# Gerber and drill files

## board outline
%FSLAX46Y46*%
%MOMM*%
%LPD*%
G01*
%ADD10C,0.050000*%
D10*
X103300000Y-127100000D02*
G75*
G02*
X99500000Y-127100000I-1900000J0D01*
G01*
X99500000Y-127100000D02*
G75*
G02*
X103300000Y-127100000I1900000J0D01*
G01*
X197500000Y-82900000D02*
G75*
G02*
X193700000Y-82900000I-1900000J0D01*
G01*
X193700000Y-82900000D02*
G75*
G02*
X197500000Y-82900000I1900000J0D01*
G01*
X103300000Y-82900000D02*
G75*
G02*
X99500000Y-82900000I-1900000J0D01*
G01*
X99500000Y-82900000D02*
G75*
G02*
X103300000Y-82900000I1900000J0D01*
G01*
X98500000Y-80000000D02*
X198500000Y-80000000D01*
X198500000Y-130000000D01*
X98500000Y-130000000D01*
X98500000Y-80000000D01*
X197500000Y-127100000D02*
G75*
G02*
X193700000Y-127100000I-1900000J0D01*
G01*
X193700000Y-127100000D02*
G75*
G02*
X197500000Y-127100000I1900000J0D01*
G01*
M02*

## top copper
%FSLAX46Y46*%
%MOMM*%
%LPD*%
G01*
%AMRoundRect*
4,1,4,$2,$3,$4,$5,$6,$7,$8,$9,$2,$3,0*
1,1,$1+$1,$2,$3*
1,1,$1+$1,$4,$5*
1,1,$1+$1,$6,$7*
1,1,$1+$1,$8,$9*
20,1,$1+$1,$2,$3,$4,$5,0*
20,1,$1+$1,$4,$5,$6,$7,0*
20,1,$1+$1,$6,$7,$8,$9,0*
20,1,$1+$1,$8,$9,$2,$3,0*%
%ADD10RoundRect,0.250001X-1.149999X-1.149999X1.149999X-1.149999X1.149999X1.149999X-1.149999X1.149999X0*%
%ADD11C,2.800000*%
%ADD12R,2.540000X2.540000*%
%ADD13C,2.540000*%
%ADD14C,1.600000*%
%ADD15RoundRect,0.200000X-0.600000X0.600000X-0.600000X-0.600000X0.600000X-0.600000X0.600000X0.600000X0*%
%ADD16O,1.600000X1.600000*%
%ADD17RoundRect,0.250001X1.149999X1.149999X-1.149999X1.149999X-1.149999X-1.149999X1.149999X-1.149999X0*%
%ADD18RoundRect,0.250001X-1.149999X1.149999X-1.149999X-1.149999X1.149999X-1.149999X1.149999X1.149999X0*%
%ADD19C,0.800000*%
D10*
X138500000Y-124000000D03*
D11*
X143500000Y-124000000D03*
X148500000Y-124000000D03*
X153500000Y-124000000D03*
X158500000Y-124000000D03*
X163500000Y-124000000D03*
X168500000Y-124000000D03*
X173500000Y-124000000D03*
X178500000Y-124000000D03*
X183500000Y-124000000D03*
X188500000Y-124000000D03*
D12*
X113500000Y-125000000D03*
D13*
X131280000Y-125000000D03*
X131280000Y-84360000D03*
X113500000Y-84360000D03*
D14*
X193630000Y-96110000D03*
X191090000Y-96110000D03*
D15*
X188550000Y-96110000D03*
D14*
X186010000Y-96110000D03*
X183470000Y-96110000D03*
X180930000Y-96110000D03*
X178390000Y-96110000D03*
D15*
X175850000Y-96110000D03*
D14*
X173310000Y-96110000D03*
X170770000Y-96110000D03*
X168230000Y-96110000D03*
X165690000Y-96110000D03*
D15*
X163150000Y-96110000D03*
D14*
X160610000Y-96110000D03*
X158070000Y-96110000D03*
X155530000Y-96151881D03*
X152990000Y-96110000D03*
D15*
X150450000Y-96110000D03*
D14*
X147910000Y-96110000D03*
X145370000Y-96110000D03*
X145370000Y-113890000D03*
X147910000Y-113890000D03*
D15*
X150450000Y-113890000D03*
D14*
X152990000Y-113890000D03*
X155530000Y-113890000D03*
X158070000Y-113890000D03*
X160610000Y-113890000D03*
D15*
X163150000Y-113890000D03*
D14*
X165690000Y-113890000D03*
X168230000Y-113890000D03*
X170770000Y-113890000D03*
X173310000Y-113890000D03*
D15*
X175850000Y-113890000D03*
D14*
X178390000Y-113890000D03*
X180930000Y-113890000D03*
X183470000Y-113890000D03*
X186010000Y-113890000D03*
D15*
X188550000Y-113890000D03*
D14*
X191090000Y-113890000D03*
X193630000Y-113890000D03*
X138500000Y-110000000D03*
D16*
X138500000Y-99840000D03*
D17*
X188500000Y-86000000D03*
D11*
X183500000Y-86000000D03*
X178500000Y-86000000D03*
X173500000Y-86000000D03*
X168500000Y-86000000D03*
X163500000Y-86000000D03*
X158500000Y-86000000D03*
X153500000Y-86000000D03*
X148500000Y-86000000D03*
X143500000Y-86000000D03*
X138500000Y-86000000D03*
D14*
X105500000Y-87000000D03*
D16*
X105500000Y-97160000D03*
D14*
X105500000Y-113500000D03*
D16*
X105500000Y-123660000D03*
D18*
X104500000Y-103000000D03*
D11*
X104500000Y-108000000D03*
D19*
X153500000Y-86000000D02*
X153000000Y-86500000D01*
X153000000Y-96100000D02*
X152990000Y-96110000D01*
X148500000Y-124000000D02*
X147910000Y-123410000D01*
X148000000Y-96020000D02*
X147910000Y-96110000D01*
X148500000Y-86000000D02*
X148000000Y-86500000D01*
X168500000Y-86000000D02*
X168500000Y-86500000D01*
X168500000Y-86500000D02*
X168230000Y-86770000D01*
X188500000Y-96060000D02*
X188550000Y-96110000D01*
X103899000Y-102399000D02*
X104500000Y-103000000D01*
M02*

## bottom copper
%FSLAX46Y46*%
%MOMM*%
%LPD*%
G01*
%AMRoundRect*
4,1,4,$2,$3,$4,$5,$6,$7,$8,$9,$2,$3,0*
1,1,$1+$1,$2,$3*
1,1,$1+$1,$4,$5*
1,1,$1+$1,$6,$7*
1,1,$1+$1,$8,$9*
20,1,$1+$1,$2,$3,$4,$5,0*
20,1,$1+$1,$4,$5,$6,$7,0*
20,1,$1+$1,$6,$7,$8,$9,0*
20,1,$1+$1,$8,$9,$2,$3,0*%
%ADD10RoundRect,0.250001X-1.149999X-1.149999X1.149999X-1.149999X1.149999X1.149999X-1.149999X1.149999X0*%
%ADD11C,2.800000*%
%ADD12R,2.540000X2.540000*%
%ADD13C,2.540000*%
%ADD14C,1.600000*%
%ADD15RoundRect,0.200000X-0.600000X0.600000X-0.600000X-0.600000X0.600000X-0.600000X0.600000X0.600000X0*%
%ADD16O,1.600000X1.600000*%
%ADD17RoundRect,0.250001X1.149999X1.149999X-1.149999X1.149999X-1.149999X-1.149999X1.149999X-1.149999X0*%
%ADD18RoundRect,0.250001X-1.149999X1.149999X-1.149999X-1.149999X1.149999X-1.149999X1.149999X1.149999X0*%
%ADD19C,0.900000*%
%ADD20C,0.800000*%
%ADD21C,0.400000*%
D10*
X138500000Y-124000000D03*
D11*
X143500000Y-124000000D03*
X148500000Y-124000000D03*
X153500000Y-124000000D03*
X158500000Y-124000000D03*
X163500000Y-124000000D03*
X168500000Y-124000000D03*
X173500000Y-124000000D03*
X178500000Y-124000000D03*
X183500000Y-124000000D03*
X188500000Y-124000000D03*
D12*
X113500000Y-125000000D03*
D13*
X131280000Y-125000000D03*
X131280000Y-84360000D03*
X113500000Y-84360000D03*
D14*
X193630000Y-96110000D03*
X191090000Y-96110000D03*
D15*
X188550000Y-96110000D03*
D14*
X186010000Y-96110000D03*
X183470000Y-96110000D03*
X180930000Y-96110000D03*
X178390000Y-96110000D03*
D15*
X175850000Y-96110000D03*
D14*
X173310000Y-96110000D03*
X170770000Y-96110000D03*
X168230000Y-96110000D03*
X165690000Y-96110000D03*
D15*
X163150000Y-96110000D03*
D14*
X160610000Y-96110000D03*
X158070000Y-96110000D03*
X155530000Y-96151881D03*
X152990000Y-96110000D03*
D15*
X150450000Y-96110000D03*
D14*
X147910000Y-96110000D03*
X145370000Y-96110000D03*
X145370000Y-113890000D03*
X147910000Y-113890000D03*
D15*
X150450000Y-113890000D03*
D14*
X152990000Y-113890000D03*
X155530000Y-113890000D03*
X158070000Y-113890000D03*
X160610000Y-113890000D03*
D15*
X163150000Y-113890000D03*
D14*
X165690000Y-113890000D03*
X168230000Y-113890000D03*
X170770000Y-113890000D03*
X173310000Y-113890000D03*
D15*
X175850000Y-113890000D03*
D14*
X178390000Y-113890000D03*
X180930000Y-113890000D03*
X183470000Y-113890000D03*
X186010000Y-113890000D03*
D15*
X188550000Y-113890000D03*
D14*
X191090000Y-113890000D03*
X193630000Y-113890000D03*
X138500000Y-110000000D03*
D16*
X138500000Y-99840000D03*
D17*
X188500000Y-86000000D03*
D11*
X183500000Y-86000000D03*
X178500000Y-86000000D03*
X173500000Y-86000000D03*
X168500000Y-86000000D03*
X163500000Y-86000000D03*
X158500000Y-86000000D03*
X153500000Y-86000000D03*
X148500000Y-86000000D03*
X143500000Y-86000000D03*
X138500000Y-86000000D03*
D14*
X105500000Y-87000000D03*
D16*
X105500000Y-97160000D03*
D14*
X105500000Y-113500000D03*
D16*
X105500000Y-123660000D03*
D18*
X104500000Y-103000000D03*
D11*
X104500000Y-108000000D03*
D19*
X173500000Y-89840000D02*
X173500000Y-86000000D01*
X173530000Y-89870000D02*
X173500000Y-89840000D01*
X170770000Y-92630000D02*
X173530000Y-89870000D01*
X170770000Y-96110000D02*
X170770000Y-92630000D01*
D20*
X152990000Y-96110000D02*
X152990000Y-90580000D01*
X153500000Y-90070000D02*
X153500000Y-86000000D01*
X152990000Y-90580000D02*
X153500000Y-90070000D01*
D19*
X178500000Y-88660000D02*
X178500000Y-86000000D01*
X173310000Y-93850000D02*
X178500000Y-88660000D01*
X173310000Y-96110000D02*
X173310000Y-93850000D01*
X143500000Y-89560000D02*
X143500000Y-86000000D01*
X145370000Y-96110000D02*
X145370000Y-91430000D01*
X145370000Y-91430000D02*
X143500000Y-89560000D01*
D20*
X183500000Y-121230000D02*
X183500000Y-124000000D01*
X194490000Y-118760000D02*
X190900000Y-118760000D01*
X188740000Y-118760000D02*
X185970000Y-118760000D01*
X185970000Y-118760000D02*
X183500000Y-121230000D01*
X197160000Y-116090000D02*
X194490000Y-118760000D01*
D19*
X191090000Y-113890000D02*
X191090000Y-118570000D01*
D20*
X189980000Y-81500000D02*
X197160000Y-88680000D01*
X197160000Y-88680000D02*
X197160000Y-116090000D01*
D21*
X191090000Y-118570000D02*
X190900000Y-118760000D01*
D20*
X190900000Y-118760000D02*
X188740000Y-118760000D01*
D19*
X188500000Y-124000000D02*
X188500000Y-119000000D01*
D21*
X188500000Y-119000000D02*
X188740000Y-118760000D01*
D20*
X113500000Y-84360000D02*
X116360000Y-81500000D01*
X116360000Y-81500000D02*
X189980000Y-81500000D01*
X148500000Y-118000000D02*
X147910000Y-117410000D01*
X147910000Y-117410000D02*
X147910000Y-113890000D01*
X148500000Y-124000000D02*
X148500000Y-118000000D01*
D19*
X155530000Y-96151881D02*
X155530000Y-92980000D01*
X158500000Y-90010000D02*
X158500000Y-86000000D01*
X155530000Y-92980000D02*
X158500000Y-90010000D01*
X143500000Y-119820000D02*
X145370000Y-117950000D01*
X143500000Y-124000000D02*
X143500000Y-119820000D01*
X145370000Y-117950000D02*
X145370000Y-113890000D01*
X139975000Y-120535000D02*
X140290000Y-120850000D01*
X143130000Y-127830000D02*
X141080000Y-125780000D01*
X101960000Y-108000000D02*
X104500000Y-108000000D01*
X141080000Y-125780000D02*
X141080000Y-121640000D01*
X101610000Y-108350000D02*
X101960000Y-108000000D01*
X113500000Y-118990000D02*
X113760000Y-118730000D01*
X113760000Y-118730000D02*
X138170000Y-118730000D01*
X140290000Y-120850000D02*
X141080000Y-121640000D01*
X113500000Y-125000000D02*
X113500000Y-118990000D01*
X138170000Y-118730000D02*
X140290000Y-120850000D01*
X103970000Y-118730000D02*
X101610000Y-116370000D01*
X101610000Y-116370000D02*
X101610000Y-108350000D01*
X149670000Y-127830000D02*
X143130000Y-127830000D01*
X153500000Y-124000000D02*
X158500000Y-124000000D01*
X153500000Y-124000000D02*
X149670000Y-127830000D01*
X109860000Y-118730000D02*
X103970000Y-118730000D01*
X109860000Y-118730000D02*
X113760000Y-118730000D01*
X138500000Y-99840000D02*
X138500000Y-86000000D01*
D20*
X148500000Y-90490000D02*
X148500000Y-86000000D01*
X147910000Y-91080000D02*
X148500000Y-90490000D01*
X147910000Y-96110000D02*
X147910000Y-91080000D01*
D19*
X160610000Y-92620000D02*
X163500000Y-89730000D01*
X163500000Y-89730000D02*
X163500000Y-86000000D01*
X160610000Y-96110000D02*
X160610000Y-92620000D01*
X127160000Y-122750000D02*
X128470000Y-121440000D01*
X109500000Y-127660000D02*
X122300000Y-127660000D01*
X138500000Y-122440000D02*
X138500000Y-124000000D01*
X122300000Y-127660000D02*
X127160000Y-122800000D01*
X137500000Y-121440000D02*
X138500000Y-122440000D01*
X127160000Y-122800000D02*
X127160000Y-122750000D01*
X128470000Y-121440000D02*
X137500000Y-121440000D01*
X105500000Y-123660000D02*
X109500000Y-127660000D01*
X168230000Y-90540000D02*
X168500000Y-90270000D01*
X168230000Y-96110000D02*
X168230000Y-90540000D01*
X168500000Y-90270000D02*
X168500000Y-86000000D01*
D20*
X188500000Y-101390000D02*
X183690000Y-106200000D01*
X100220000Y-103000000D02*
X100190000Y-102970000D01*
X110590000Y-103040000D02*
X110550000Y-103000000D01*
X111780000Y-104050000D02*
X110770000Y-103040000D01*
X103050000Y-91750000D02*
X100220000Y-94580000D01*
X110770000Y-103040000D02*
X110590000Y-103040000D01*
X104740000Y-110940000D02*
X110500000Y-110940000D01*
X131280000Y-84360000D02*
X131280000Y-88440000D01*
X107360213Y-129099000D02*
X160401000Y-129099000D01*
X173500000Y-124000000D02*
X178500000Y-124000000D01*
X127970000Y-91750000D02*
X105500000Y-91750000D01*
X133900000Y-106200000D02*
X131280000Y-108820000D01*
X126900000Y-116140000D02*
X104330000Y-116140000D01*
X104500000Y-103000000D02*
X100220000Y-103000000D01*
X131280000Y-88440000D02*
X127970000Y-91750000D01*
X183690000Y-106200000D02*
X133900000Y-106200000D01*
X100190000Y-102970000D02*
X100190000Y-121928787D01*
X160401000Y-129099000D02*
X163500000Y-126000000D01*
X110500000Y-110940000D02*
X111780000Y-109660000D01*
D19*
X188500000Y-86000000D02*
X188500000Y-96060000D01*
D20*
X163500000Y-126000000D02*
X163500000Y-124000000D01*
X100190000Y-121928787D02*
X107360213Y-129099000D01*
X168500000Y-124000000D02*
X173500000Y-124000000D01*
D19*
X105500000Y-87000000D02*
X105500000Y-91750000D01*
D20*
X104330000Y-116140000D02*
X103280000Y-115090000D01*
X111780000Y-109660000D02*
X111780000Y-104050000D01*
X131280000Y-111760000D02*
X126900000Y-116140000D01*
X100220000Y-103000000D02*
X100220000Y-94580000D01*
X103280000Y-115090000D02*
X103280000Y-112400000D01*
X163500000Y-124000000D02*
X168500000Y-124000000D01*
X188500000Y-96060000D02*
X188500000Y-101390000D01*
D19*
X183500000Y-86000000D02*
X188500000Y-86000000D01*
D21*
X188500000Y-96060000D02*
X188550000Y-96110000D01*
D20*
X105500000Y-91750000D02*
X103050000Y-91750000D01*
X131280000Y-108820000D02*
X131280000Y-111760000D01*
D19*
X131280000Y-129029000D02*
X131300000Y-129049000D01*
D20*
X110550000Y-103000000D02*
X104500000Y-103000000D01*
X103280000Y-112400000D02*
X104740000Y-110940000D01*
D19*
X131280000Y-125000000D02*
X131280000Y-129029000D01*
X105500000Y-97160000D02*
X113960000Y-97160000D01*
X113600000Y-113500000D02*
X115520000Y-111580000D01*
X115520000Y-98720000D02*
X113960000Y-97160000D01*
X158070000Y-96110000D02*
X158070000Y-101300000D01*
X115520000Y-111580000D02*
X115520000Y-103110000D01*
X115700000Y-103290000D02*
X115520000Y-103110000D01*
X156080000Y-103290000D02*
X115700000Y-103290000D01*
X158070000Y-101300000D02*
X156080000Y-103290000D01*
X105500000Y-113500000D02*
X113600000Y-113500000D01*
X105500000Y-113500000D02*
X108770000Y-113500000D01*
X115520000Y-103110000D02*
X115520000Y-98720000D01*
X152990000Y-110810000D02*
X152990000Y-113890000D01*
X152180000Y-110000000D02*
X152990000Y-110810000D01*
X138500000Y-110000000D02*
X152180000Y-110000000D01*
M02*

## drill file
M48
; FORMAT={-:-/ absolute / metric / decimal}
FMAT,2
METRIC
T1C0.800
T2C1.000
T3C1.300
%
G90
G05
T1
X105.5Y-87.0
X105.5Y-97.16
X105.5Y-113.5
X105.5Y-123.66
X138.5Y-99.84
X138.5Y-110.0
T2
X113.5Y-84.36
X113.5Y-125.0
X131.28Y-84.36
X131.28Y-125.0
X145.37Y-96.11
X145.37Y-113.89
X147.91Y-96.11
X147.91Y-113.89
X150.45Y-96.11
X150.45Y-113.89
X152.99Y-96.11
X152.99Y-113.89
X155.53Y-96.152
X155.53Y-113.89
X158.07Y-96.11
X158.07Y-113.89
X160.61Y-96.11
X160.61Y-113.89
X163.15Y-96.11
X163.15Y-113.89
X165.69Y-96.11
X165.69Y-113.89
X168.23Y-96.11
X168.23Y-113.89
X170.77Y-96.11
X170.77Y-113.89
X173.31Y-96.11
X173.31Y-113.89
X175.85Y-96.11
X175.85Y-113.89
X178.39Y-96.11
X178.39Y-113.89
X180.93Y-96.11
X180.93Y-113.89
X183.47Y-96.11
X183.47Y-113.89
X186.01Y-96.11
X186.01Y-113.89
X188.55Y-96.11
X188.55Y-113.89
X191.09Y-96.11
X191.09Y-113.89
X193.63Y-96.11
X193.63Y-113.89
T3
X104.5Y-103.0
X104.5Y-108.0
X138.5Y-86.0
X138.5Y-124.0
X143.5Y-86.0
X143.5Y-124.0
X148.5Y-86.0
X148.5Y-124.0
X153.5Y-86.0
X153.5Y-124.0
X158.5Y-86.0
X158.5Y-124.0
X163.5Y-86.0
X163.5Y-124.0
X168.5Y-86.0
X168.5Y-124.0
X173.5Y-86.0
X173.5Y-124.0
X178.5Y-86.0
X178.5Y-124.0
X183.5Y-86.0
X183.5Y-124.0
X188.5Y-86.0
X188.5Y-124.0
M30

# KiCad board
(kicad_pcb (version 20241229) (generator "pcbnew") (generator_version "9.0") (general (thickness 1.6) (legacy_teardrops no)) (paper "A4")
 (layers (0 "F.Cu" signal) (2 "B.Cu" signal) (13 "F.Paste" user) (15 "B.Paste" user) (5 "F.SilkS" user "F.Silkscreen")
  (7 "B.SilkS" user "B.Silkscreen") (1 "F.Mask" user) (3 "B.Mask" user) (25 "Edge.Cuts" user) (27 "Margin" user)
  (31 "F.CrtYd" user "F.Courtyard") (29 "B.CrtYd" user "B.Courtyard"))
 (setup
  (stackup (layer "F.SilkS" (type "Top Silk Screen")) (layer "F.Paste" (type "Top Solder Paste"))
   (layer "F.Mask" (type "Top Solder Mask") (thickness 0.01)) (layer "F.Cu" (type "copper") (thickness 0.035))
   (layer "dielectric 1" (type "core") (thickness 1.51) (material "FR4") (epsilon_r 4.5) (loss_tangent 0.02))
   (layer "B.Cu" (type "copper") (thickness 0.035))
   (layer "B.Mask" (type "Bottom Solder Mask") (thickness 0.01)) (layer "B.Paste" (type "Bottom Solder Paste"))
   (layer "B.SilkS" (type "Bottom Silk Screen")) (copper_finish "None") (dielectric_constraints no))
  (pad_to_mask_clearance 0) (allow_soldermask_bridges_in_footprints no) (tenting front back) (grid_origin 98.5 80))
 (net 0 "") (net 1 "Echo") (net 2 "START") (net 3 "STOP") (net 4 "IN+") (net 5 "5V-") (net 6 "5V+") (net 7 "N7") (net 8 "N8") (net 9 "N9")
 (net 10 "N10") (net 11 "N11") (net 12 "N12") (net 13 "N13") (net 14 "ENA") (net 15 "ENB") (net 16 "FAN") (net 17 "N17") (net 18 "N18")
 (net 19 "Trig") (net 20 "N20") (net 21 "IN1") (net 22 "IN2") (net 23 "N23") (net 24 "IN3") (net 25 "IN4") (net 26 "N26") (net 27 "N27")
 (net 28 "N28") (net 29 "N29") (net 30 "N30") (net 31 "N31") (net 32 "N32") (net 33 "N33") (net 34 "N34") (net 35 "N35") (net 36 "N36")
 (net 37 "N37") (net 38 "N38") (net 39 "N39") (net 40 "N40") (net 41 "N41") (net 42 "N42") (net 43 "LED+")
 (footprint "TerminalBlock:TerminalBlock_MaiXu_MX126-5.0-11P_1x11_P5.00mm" (layer "F.Cu") (at 138.5 124)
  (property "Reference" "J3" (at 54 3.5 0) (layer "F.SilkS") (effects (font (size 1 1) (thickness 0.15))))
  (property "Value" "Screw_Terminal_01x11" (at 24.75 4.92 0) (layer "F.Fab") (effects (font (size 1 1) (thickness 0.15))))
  (pad "1" thru_hole roundrect (at 0 0) (size 2.8 2.8) (drill 1.3) (layers "*.Cu" "*.Mask") (remove_unused_layers no)
   (roundrect_rratio 0.089286) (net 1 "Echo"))
  (pad "2" thru_hole circle (at 5 0) (size 2.8 2.8) (drill 1.3) (layers "*.Cu" "*.Mask") (remove_unused_layers no) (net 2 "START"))
  (pad "3" thru_hole circle (at 10 0) (size 2.8 2.8) (drill 1.3) (layers "*.Cu" "*.Mask") (remove_unused_layers no) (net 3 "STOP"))
  (pad "4" thru_hole circle (at 15 0) (size 2.8 2.8) (drill 1.3) (layers "*.Cu" "*.Mask") (remove_unused_layers no) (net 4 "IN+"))
  (pad "5" thru_hole circle (at 20 0) (size 2.8 2.8) (drill 1.3) (layers "*.Cu" "*.Mask") (remove_unused_layers no) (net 4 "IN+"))
  (pad "6" thru_hole circle (at 25 0) (size 2.8 2.8) (drill 1.3) (layers "*.Cu" "*.Mask") (remove_unused_layers no) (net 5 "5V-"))
  (pad "7" thru_hole circle (at 30 0) (size 2.8 2.8) (drill 1.3) (layers "*.Cu" "*.Mask") (remove_unused_layers no) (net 5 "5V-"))
  (pad "8" thru_hole circle (at 35 0) (size 2.8 2.8) (drill 1.3) (layers "*.Cu" "*.Mask") (remove_unused_layers no) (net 5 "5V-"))
  (pad "9" thru_hole circle (at 40 0) (size 2.8 2.8) (drill 1.3) (layers "*.Cu" "*.Mask") (remove_unused_layers no) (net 5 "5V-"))
  (pad "10" thru_hole circle (at 45 0) (size 2.8 2.8) (drill 1.3) (layers "*.Cu" "*.Mask") (remove_unused_layers no) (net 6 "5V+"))
  (pad "11" thru_hole circle (at 50 0) (size 2.8 2.8) (drill 1.3) (layers "*.Cu" "*.Mask") (remove_unused_layers no) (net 6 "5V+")))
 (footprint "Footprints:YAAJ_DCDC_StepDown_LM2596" (layer "F.Cu") (at 113.5 125 90)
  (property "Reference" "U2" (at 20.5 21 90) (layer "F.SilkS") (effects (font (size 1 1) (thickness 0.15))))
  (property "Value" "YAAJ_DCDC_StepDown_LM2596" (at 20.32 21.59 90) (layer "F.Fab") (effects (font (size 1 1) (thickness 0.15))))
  (pad "1" thru_hole rect (at 0 0 90) (size 2.54 2.54) (drill 1) (layers "*.Cu" "*.Mask") (remove_unused_layers no) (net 4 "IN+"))
  (pad "2" thru_hole circle (at 0 17.78 90) (size 2.54 2.54) (drill 1) (layers "*.Cu" "*.Mask") (remove_unused_layers no) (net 5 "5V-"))
  (pad "3" thru_hole circle (at 40.64 17.78 90) (size 2.54 2.54) (drill 1) (layers "*.Cu" "*.Mask") (remove_unused_layers no) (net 5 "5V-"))
  (pad "4" thru_hole circle (at 40.64 0 90) (size 2.54 2.54) (drill 1) (layers "*.Cu" "*.Mask") (remove_unused_layers no) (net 6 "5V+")))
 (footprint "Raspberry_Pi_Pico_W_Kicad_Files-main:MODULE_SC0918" (layer "F.Cu") (at 169.5 105 -90)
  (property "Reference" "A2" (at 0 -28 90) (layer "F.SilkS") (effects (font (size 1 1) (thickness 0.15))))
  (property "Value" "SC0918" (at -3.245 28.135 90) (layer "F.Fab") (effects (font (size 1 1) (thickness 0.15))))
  (pad "1" thru_hole circle (at -8.89 -24.13 270) (size 1.6 1.6) (drill 1) (layers "*.Cu" "*.Mask") (remove_unused_layers no) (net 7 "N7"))
  (pad "2" thru_hole circle (at -8.89 -21.59 270) (size 1.6 1.6) (drill 1) (layers "*.Cu" "*.Mask") (remove_unused_layers no) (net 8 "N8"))
  (pad "3" thru_hole roundrect (at -8.89 -19.05 270) (size 1.6 1.6) (drill 1) (layers "*.Cu" "*.Mask") (remove_unused_layers no)
   (roundrect_rratio 0.125) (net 5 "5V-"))
  (pad "4" thru_hole circle (at -8.89 -16.51 270) (size 1.6 1.6) (drill 1) (layers "*.Cu" "*.Mask") (remove_unused_layers no) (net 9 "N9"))
  (pad "5" thru_hole circle (at -8.89 -13.97 270) (size 1.6 1.6) (drill 1) (layers "*.Cu" "*.Mask") (remove_unused_layers no) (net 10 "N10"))
  (pad "6" thru_hole circle (at -8.89 -11.43 270) (size 1.6 1.6) (drill 1) (layers "*.Cu" "*.Mask") (remove_unused_layers no) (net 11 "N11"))
  (pad "7" thru_hole circle (at -8.89 -8.89 270) (size 1.6 1.6) (drill 1) (layers "*.Cu" "*.Mask") (remove_unused_layers no) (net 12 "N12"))
  (pad "8" thru_hole roundrect (at -8.89 -6.35 270) (size 1.6 1.6) (drill 1) (layers "*.Cu" "*.Mask") (remove_unused_layers no)
   (roundrect_rratio 0.125) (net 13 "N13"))
  (pad "9" thru_hole circle (at -8.89 -3.81 270) (size 1.6 1.6) (drill 1) (layers "*.Cu" "*.Mask") (remove_unused_layers no) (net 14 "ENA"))
  (pad "10" thru_hole circle (at -8.89 -1.27 270) (size 1.6 1.6) (drill 1) (layers "*.Cu" "*.Mask") (remove_unused_layers no) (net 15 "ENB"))
  (pad "11" thru_hole circle (at -8.89 1.27 270) (size 1.6 1.6) (drill 1) (layers "*.Cu" "*.Mask") (remove_unused_layers no) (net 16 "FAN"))
  (pad "12" thru_hole circle (at -8.89 3.81 270) (size 1.6 1.6) (drill 1) (layers "*.Cu" "*.Mask") (remove_unused_layers no) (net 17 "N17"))
  (pad "13" thru_hole roundrect (at -8.89 6.35 270) (size 1.6 1.6) (drill 1) (layers "*.Cu" "*.Mask") (remove_unused_layers no)
   (roundrect_rratio 0.125) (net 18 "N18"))
  (pad "14" thru_hole circle (at -8.89 8.89 270) (size 1.6 1.6) (drill 1) (layers "*.Cu" "*.Mask") (remove_unused_layers no) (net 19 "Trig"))
  (pad "15" thru_hole circle (at -8.89 11.43 270) (size 1.6 1.6) (drill 1) (layers "*.Cu" "*.Mask") (remove_unused_layers no) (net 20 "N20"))
  (pad "16" thru_hole circle (at -8.848119 13.97 270) (size 1.6 1.6) (drill 1) (layers "*.Cu" "*.Mask") (remove_unused_layers no)
   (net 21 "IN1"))
  (pad "17" thru_hole circle (at -8.89 16.51 270) (size 1.6 1.6) (drill 1) (layers "*.Cu" "*.Mask") (remove_unused_layers no) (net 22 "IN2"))
  (pad "18" thru_hole roundrect (at -8.89 19.05 270) (size 1.6 1.6) (drill 1) (layers "*.Cu" "*.Mask") (remove_unused_layers no)
   (roundrect_rratio 0.125) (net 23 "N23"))
  (pad "19" thru_hole circle (at -8.89 21.59 270) (size 1.6 1.6) (drill 1) (layers "*.Cu" "*.Mask") (remove_unused_layers no) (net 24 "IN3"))
  (pad "20" thru_hole circle (at -8.89 24.13 270) (size 1.6 1.6) (drill 1) (layers "*.Cu" "*.Mask") (remove_unused_layers no) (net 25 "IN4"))
  (pad "21" thru_hole circle (at 8.89 24.13 270) (size 1.6 1.6) (drill 1) (layers "*.Cu" "*.Mask") (remove_unused_layers no) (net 2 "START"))
  (pad "22" thru_hole circle (at 8.89 21.59 270) (size 1.6 1.6) (drill 1) (layers "*.Cu" "*.Mask") (remove_unused_layers no) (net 3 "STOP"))
  (pad "23" thru_hole roundrect (at 8.89 19.05 270) (size 1.6 1.6) (drill 1) (layers "*.Cu" "*.Mask") (remove_unused_layers no)
   (roundrect_rratio 0.125) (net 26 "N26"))
  (pad "24" thru_hole circle (at 8.89 16.51 270) (size 1.6 1.6) (drill 1) (layers "*.Cu" "*.Mask") (remove_unused_layers no) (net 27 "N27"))
  (pad "25" thru_hole circle (at 8.89 13.97 270) (size 1.6 1.6) (drill 1) (layers "*.Cu" "*.Mask") (remove_unused_layers no) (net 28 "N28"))
  (pad "26" thru_hole circle (at 8.89 11.43 270) (size 1.6 1.6) (drill 1) (layers "*.Cu" "*.Mask") (remove_unused_layers no) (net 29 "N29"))
  (pad "27" thru_hole circle (at 8.89 8.89 270) (size 1.6 1.6) (drill 1) (layers "*.Cu" "*.Mask") (remove_unused_layers no) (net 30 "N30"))
  (pad "28" thru_hole roundrect (at 8.89 6.35 270) (size 1.6 1.6) (drill 1) (layers "*.Cu" "*.Mask") (remove_unused_layers no)
   (roundrect_rratio 0.125) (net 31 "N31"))
  (pad "29" thru_hole circle (at 8.89 3.81 270) (size 1.6 1.6) (drill 1) (layers "*.Cu" "*.Mask") (remove_unused_layers no) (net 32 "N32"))
  (pad "30" thru_hole circle (at 8.89 1.27 270) (size 1.6 1.6) (drill 1) (layers "*.Cu" "*.Mask") (remove_unused_layers no) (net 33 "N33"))
  (pad "31" thru_hole circle (at 8.89 -1.27 270) (size 1.6 1.6) (drill 1) (layers "*.Cu" "*.Mask") (remove_unused_layers no) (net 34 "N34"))
  (pad "32" thru_hole circle (at 8.89 -3.81 270) (size 1.6 1.6) (drill 1) (layers "*.Cu" "*.Mask") (remove_unused_layers no) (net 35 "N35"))
  (pad "33" thru_hole roundrect (at 8.89 -6.35 270) (size 1.6 1.6) (drill 1) (layers "*.Cu" "*.Mask") (remove_unused_layers no)
   (roundrect_rratio 0.125) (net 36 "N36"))
  (pad "34" thru_hole circle (at 8.89 -8.89 270) (size 1.6 1.6) (drill 1) (layers "*.Cu" "*.Mask") (remove_unused_layers no) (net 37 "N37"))
  (pad "35" thru_hole circle (at 8.89 -11.43 270) (size 1.6 1.6) (drill 1) (layers "*.Cu" "*.Mask") (remove_unused_layers no) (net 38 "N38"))
  (pad "36" thru_hole circle (at 8.89 -13.97 270) (size 1.6 1.6) (drill 1) (layers "*.Cu" "*.Mask") (remove_unused_layers no) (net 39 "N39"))
  (pad "37" thru_hole circle (at 8.89 -16.51 270) (size 1.6 1.6) (drill 1) (layers "*.Cu" "*.Mask") (remove_unused_layers no) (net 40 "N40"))
  (pad "38" thru_hole roundrect (at 8.89 -19.05 270) (size 1.6 1.6) (drill 1) (layers "*.Cu" "*.Mask") (remove_unused_layers no)
   (roundrect_rratio 0.125) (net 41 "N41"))
  (pad "39" thru_hole circle (at 8.89 -21.59 270) (size 1.6 1.6) (drill 1) (layers "*.Cu" "*.Mask") (remove_unused_layers no) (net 6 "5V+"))
  (pad "40" thru_hole circle (at 8.89 -24.13 270) (size 1.6 1.6) (drill 1) (layers "*.Cu" "*.Mask") (remove_unused_layers no) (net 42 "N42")))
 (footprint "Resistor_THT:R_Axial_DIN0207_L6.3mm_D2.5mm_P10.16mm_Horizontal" (layer "F.Cu") (at 138.5 110 90)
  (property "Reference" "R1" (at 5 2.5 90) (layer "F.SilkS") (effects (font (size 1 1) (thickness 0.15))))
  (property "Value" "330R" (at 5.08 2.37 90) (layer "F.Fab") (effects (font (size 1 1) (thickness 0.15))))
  (pad "1" thru_hole circle (at 0 0 90) (size 1.6 1.6) (drill 0.8) (layers "*.Cu" "*.Mask") (remove_unused_layers no) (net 27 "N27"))
  (pad "2" thru_hole oval (at 10.16 0 90) (size 1.6 1.6) (drill 0.8) (layers "*.Cu" "*.Mask") (remove_unused_layers no) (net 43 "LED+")))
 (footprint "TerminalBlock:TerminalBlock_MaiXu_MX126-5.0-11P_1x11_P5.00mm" (layer "F.Cu") (at 188.5 86 180)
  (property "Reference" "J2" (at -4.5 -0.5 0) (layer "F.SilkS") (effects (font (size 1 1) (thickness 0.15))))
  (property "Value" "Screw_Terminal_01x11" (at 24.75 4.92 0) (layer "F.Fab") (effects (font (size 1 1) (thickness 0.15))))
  (pad "1" thru_hole roundrect (at 0 0 180) (size 2.8 2.8) (drill 1.3) (layers "*.Cu" "*.Mask") (remove_unused_layers no)
   (roundrect_rratio 0.089286) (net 5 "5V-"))
  (pad "2" thru_hole circle (at 5 0 180) (size 2.8 2.8) (drill 1.3) (layers "*.Cu" "*.Mask") (remove_unused_layers no) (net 5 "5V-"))
  (pad "3" thru_hole circle (at 10 0 180) (size 2.8 2.8) (drill 1.3) (layers "*.Cu" "*.Mask") (remove_unused_layers no) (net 14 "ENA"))
  (pad "4" thru_hole circle (at 15 0 180) (size 2.8 2.8) (drill 1.3) (layers "*.Cu" "*.Mask") (remove_unused_layers no) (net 15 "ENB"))
  (pad "5" thru_hole circle (at 20 0 180) (size 2.8 2.8) (drill 1.3) (layers "*.Cu" "*.Mask") (remove_unused_layers no) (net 16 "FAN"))
  (pad "6" thru_hole circle (at 25 0 180) (size 2.8 2.8) (drill 1.3) (layers "*.Cu" "*.Mask") (remove_unused_layers no) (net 19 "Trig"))
  (pad "7" thru_hole circle (at 30 0 180) (size 2.8 2.8) (drill 1.3) (layers "*.Cu" "*.Mask") (remove_unused_layers no) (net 21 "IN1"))
  (pad "8" thru_hole circle (at 35 0 180) (size 2.8 2.8) (drill 1.3) (layers "*.Cu" "*.Mask") (remove_unused_layers no) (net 22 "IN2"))
  (pad "9" thru_hole circle (at 40 0 180) (size 2.8 2.8) (drill 1.3) (layers "*.Cu" "*.Mask") (remove_unused_layers no) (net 24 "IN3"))
  (pad "10" thru_hole circle (at 45 0 180) (size 2.8 2.8) (drill 1.3) (layers "*.Cu" "*.Mask") (remove_unused_layers no) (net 25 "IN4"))
  (pad "11" thru_hole circle (at 50 0 180) (size 2.8 2.8) (drill 1.3) (layers "*.Cu" "*.Mask") (remove_unused_layers no) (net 43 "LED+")))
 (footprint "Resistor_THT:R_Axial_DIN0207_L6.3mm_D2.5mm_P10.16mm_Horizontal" (layer "F.Cu") (at 105.5 87 -90)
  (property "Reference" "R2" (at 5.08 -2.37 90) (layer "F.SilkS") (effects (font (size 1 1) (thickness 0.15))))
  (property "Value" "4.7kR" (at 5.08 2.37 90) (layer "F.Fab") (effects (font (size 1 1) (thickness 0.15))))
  (pad "1" thru_hole circle (at 0 0 270) (size 1.6 1.6) (drill 0.8) (layers "*.Cu" "*.Mask") (remove_unused_layers no) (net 5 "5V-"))
  (pad "2" thru_hole oval (at 10.16 0 270) (size 1.6 1.6) (drill 0.8) (layers "*.Cu" "*.Mask") (remove_unused_layers no) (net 20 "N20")))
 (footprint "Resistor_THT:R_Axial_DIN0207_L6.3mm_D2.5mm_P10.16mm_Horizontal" (layer "F.Cu") (at 105.5 113.5 -90)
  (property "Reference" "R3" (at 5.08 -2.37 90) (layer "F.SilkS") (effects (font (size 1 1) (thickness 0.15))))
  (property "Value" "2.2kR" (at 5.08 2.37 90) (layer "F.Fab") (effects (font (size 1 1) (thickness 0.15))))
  (pad "1" thru_hole circle (at 0 0 270) (size 1.6 1.6) (drill 0.8) (layers "*.Cu" "*.Mask") (remove_unused_layers no) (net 20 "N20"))
  (pad "2" thru_hole oval (at 10.16 0 270) (size 1.6 1.6) (drill 0.8) (layers "*.Cu" "*.Mask") (remove_unused_layers no) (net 1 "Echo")))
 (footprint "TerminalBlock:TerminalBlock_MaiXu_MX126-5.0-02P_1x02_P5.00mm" (layer "F.Cu") (at 104.5 103 -90)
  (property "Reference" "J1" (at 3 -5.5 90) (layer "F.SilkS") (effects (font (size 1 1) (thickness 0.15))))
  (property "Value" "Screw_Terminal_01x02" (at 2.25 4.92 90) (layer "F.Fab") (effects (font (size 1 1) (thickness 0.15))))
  (pad "1" thru_hole roundrect (at 0 0 270) (size 2.8 2.8) (drill 1.3) (layers "*.Cu" "*.Mask") (remove_unused_layers no)
   (roundrect_rratio 0.089286) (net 5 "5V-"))
  (pad "2" thru_hole circle (at 5 0 270) (size 2.8 2.8) (drill 1.3) (layers "*.Cu" "*.Mask") (remove_unused_layers no) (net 4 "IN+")))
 (gr_circle (center 101.4 127.1) (end 103.3 127.1) (stroke (width 0.05) (type solid)) (fill no) (layer "Edge.Cuts"))
 (gr_circle (center 195.6 82.9) (end 197.5 82.9) (stroke (width 0.05) (type solid)) (fill no) (layer "Edge.Cuts"))
 (gr_circle (center 101.4 82.9) (end 103.3 82.9) (stroke (width 0.05) (type solid)) (fill no) (layer "Edge.Cuts"))
 (gr_rect (start 98.5 80) (end 198.5 130) (stroke (width 0.05) (type solid)) (fill no) (locked yes) (layer "Edge.Cuts"))
 (gr_circle (center 195.6 127.1) (end 197.5 127.1) (stroke (width 0.05) (type solid)) (fill no) (layer "Edge.Cuts"))
 (segment (start 173.5 89.84) (end 173.5 86) (width 0.9) (layer "B.Cu") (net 15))
 (segment (start 173.53 89.87) (end 173.5 89.84) (width 0.9) (layer "B.Cu") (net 15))
 (segment (start 170.77 92.63) (end 173.53 89.87) (width 0.9) (layer "B.Cu") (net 15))
 (segment (start 170.77 96.11) (end 170.77 92.63) (width 0.9) (layer "B.Cu") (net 15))
 (segment (start 153.5 86) (end 153 86.5) (width 0.8) (layer "F.Cu") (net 22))
 (segment (start 153 96.1) (end 152.99 96.11) (width 0.8) (layer "F.Cu") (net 22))
 (segment (start 152.99 96.11) (end 152.99 90.58) (width 0.8) (layer "B.Cu") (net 22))
 (segment (start 153.5 90.07) (end 153.5 86) (width 0.8) (layer "B.Cu") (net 22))
 (segment (start 152.99 90.58) (end 153.5 90.07) (width 0.8) (layer "B.Cu") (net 22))
 (segment (start 178.5 88.66) (end 178.5 86) (width 0.9) (layer "B.Cu") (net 14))
 (segment (start 173.31 93.85) (end 178.5 88.66) (width 0.9) (layer "B.Cu") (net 14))
 (segment (start 173.31 96.11) (end 173.31 93.85) (width 0.9) (layer "B.Cu") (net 14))
 (segment (start 143.5 89.56) (end 143.5 86) (width 0.9) (layer "B.Cu") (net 25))
 (segment (start 145.37 96.11) (end 145.37 91.43) (width 0.9) (layer "B.Cu") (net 25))
 (segment (start 145.37 91.43) (end 143.5 89.56) (width 0.9) (layer "B.Cu") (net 25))
 (segment (start 183.5 121.23) (end 183.5 124) (width 0.8) (layer "B.Cu") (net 6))
 (segment (start 194.49 118.76) (end 190.9 118.76) (width 0.8) (layer "B.Cu") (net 6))
 (segment (start 188.74 118.76) (end 185.97 118.76) (width 0.8) (layer "B.Cu") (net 6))
 (segment (start 185.97 118.76) (end 183.5 121.23) (width 0.8) (layer "B.Cu") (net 6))
 (segment (start 197.16 116.09) (end 194.49 118.76) (width 0.8) (layer "B.Cu") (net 6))
 (segment (start 191.09 113.89) (end 191.09 118.57) (width 0.9) (layer "B.Cu") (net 6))
 (segment (start 189.98 81.5) (end 197.16 88.68) (width 0.8) (layer "B.Cu") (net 6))
 (segment (start 197.16 88.68) (end 197.16 116.09) (width 0.8) (layer "B.Cu") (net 6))
 (segment (start 191.09 118.57) (end 190.9 118.76) (width 0.4) (layer "B.Cu") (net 6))
 (segment (start 190.9 118.76) (end 188.74 118.76) (width 0.8) (layer "B.Cu") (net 6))
 (segment (start 188.5 124) (end 188.5 119) (width 0.9) (layer "B.Cu") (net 6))
 (segment (start 188.5 119) (end 188.74 118.76) (width 0.4) (layer "B.Cu") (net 6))
 (segment (start 113.5 84.36) (end 116.36 81.5) (width 0.8) (layer "B.Cu") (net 6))
 (segment (start 116.36 81.5) (end 189.98 81.5) (width 0.8) (layer "B.Cu") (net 6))
 (segment (start 148.5 124) (end 147.91 123.41) (width 0.8) (layer "F.Cu") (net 3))
 (segment (start 148.5 118) (end 147.91 117.41) (width 0.8) (layer "B.Cu") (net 3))
 (segment (start 147.91 117.41) (end 147.91 113.89) (width 0.8) (layer "B.Cu") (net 3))
 (segment (start 148.5 124) (end 148.5 118) (width 0.8) (layer "B.Cu") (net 3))
 (segment (start 155.53 96.151881) (end 155.53 92.98) (width 0.9) (layer "B.Cu") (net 21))
 (segment (start 158.5 90.01) (end 158.5 86) (width 0.9) (layer "B.Cu") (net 21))
 (segment (start 155.53 92.98) (end 158.5 90.01) (width 0.9) (layer "B.Cu") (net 21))
 (segment (start 143.5 119.82) (end 145.37 117.95) (width 0.9) (layer "B.Cu") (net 2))
 (segment (start 143.5 124) (end 143.5 119.82) (width 0.9) (layer "B.Cu") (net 2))
 (segment (start 145.37 117.95) (end 145.37 113.89) (width 0.9) (layer "B.Cu") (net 2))
 (segment (start 139.975 120.535) (end 140.29 120.85) (width 0.9) (layer "B.Cu") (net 4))
 (segment (start 143.13 127.83) (end 141.08 125.78) (width 0.9) (layer "B.Cu") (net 4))
 (segment (start 101.96 108) (end 104.5 108) (width 0.9) (layer "B.Cu") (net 4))
 (segment (start 141.08 125.78) (end 141.08 121.64) (width 0.9) (layer "B.Cu") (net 4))
 (segment (start 101.61 108.35) (end 101.96 108) (width 0.9) (layer "B.Cu") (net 4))
 (segment (start 113.5 118.99) (end 113.76 118.73) (width 0.9) (layer "B.Cu") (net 4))
 (segment (start 113.76 118.73) (end 138.17 118.73) (width 0.9) (layer "B.Cu") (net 4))
 (segment (start 140.29 120.85) (end 141.08 121.64) (width 0.9) (layer "B.Cu") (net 4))
 (segment (start 113.5 125) (end 113.5 118.99) (width 0.9) (layer "B.Cu") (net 4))
 (segment (start 138.17 118.73) (end 140.29 120.85) (width 0.9) (layer "B.Cu") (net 4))
 (segment (start 103.97 118.73) (end 101.61 116.37) (width 0.9) (layer "B.Cu") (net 4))
 (segment (start 101.61 116.37) (end 101.61 108.35) (width 0.9) (layer "B.Cu") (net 4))
 (segment (start 149.67 127.83) (end 143.13 127.83) (width 0.9) (layer "B.Cu") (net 4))
 (segment (start 153.5 124) (end 158.5 124) (width 0.9) (layer "B.Cu") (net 4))
 (segment (start 153.5 124) (end 149.67 127.83) (width 0.9) (layer "B.Cu") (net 4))
 (segment (start 109.86 118.73) (end 103.97 118.73) (width 0.9) (layer "B.Cu") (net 4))
 (segment (start 109.86 118.73) (end 113.76 118.73) (width 0.9) (layer "B.Cu") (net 4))
 (segment (start 138.5 99.84) (end 138.5 86) (width 0.9) (layer "B.Cu") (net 43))
 (segment (start 148 96.02) (end 147.91 96.11) (width 0.8) (layer "F.Cu") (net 24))
 (segment (start 148.5 86) (end 148 86.5) (width 0.8) (layer "F.Cu") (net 24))
 (segment (start 148.5 90.49) (end 148.5 86) (width 0.8) (layer "B.Cu") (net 24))
 (segment (start 147.91 91.08) (end 148.5 90.49) (width 0.8) (layer "B.Cu") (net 24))
 (segment (start 147.91 96.11) (end 147.91 91.08) (width 0.8) (layer "B.Cu") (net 24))
 (segment (start 160.61 92.62) (end 163.5 89.73) (width 0.9) (layer "B.Cu") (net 19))
 (segment (start 163.5 89.73) (end 163.5 86) (width 0.9) (layer "B.Cu") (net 19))
 (segment (start 160.61 96.11) (end 160.61 92.62) (width 0.9) (layer "B.Cu") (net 19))
 (segment (start 127.16 122.75) (end 128.47 121.44) (width 0.9) (layer "B.Cu") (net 1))
 (segment (start 109.5 127.66) (end 122.3 127.66) (width 0.9) (layer "B.Cu") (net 1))
 (segment (start 138.5 122.44) (end 138.5 124) (width 0.9) (layer "B.Cu") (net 1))
 (segment (start 122.3 127.66) (end 127.16 122.8) (width 0.9) (layer "B.Cu") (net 1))
 (segment (start 137.5 121.44) (end 138.5 122.44) (width 0.9) (layer "B.Cu") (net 1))
 (segment (start 127.16 122.8) (end 127.16 122.75) (width 0.9) (layer "B.Cu") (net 1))
 (segment (start 128.47 121.44) (end 137.5 121.44) (width 0.9) (layer "B.Cu") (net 1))
 (segment (start 105.5 123.66) (end 109.5 127.66) (width 0.9) (layer "B.Cu") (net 1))
 (segment (start 168.5 86) (end 168.5 86.5) (width 0.8) (layer "F.Cu") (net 16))
 (segment (start 168.5 86.5) (end 168.23 86.77) (width 0.8) (layer "F.Cu") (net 16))
 (segment (start 168.23 90.54) (end 168.5 90.27) (width 0.9) (layer "B.Cu") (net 16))
 (segment (start 168.23 96.11) (end 168.23 90.54) (width 0.9) (layer "B.Cu") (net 16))
 (segment (start 168.5 90.27) (end 168.5 86) (width 0.9) (layer "B.Cu") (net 16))
 (segment (start 188.5 96.06) (end 188.55 96.11) (width 0.8) (layer "F.Cu") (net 5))
 (segment (start 103.899 102.399) (end 104.5 103) (width 0.8) (layer "F.Cu") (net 5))
 (segment (start 188.5 101.39) (end 183.69 106.2) (width 0.8) (layer "B.Cu") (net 5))
 (segment (start 100.22 103) (end 100.19 102.97) (width 0.8) (layer "B.Cu") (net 5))
 (segment (start 110.59 103.04) (end 110.55 103) (width 0.8) (layer "B.Cu") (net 5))
 (segment (start 111.78 104.05) (end 110.77 103.04) (width 0.8) (layer "B.Cu") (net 5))
 (segment (start 103.05 91.75) (end 100.22 94.58) (width 0.8) (layer "B.Cu") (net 5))
 (segment (start 110.77 103.04) (end 110.59 103.04) (width 0.8) (layer "B.Cu") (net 5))
 (segment (start 104.74 110.94) (end 110.5 110.94) (width 0.8) (layer "B.Cu") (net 5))
 (segment (start 131.28 84.36) (end 131.28 88.44) (width 0.8) (layer "B.Cu") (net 5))
 (segment (start 107.360213 129.099) (end 160.401 129.099) (width 0.8) (layer "B.Cu") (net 5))
 (segment (start 173.5 124) (end 178.5 124) (width 0.8) (layer "B.Cu") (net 5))
 (segment (start 127.97 91.75) (end 105.5 91.75) (width 0.8) (layer "B.Cu") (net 5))
 (segment (start 133.9 106.2) (end 131.28 108.82) (width 0.8) (layer "B.Cu") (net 5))
 (segment (start 126.9 116.14) (end 104.33 116.14) (width 0.8) (layer "B.Cu") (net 5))
 (segment (start 104.5 103) (end 100.22 103) (width 0.8) (layer "B.Cu") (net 5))
 (segment (start 131.28 88.44) (end 127.97 91.75) (width 0.8) (layer "B.Cu") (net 5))
 (segment (start 183.69 106.2) (end 133.9 106.2) (width 0.8) (layer "B.Cu") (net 5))
 (segment (start 100.19 102.97) (end 100.19 121.928787) (width 0.8) (layer "B.Cu") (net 5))
 (segment (start 160.401 129.099) (end 163.5 126) (width 0.8) (layer "B.Cu") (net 5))
 (segment (start 110.5 110.94) (end 111.78 109.66) (width 0.8) (layer "B.Cu") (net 5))
 (segment (start 188.5 86) (end 188.5 96.06) (width 0.9) (layer "B.Cu") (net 5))
 (segment (start 163.5 126) (end 163.5 124) (width 0.8) (layer "B.Cu") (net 5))
 (segment (start 100.19 121.928787) (end 107.360213 129.099) (width 0.8) (layer "B.Cu") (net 5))
 (segment (start 168.5 124) (end 173.5 124) (width 0.8) (layer "B.Cu") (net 5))
 (segment (start 105.5 87) (end 105.5 91.75) (width 0.9) (layer "B.Cu") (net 5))
 (segment (start 104.33 116.14) (end 103.28 115.09) (width 0.8) (layer "B.Cu") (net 5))
 (segment (start 111.78 109.66) (end 111.78 104.05) (width 0.8) (layer "B.Cu") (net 5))
 (segment (start 131.28 111.76) (end 126.9 116.14) (width 0.8) (layer "B.Cu") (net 5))
 (segment (start 100.22 103) (end 100.22 94.58) (width 0.8) (layer "B.Cu") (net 5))
 (segment (start 103.28 115.09) (end 103.28 112.4) (width 0.8) (layer "B.Cu") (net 5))
 (segment (start 163.5 124) (end 168.5 124) (width 0.8) (layer "B.Cu") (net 5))
 (segment (start 188.5 96.06) (end 188.5 101.39) (width 0.8) (layer "B.Cu") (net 5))
 (segment (start 183.5 86) (end 188.5 86) (width 0.9) (layer "B.Cu") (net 5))
 (segment (start 188.5 96.06) (end 188.55 96.11) (width 0.4) (layer "B.Cu") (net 5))
 (segment (start 105.5 91.75) (end 103.05 91.75) (width 0.8) (layer "B.Cu") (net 5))
 (segment (start 131.28 108.82) (end 131.28 111.76) (width 0.8) (layer "B.Cu") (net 5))
 (segment (start 131.28 129.029) (end 131.3 129.049) (width 0.9) (layer "B.Cu") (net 5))
 (segment (start 110.55 103) (end 104.5 103) (width 0.8) (layer "B.Cu") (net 5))
 (segment (start 103.28 112.4) (end 104.74 110.94) (width 0.8) (layer "B.Cu") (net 5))
 (segment (start 131.28 125) (end 131.28 129.029) (width 0.9) (layer "B.Cu") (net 5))
 (segment (start 105.5 97.16) (end 113.96 97.16) (width 0.9) (layer "B.Cu") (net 20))
 (segment (start 113.6 113.5) (end 115.52 111.58) (width 0.9) (layer "B.Cu") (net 20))
 (segment (start 115.52 98.72) (end 113.96 97.16) (width 0.9) (layer "B.Cu") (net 20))
 (segment (start 158.07 96.11) (end 158.07 101.3) (width 0.9) (layer "B.Cu") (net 20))
 (segment (start 115.52 111.58) (end 115.52 103.11) (width 0.9) (layer "B.Cu") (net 20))
 (segment (start 115.7 103.29) (end 115.52 103.11) (width 0.9) (layer "B.Cu") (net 20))
 (segment (start 156.08 103.29) (end 115.7 103.29) (width 0.9) (layer "B.Cu") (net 20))
 (segment (start 158.07 101.3) (end 156.08 103.29) (width 0.9) (layer "B.Cu") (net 20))
 (segment (start 105.5 113.5) (end 113.6 113.5) (width 0.9) (layer "B.Cu") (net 20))
 (segment (start 105.5 113.5) (end 108.77 113.5) (width 0.9) (layer "B.Cu") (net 20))
 (segment (start 115.52 103.11) (end 115.52 98.72) (width 0.9) (layer "B.Cu") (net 20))
 (segment (start 152.99 110.81) (end 152.99 113.89) (width 0.9) (layer "B.Cu") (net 27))
 (segment (start 152.18 110) (end 152.99 110.81) (width 0.9) (layer "B.Cu") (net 27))
 (segment (start 138.5 110) (end 152.18 110) (width 0.9) (layer "B.Cu") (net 27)))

